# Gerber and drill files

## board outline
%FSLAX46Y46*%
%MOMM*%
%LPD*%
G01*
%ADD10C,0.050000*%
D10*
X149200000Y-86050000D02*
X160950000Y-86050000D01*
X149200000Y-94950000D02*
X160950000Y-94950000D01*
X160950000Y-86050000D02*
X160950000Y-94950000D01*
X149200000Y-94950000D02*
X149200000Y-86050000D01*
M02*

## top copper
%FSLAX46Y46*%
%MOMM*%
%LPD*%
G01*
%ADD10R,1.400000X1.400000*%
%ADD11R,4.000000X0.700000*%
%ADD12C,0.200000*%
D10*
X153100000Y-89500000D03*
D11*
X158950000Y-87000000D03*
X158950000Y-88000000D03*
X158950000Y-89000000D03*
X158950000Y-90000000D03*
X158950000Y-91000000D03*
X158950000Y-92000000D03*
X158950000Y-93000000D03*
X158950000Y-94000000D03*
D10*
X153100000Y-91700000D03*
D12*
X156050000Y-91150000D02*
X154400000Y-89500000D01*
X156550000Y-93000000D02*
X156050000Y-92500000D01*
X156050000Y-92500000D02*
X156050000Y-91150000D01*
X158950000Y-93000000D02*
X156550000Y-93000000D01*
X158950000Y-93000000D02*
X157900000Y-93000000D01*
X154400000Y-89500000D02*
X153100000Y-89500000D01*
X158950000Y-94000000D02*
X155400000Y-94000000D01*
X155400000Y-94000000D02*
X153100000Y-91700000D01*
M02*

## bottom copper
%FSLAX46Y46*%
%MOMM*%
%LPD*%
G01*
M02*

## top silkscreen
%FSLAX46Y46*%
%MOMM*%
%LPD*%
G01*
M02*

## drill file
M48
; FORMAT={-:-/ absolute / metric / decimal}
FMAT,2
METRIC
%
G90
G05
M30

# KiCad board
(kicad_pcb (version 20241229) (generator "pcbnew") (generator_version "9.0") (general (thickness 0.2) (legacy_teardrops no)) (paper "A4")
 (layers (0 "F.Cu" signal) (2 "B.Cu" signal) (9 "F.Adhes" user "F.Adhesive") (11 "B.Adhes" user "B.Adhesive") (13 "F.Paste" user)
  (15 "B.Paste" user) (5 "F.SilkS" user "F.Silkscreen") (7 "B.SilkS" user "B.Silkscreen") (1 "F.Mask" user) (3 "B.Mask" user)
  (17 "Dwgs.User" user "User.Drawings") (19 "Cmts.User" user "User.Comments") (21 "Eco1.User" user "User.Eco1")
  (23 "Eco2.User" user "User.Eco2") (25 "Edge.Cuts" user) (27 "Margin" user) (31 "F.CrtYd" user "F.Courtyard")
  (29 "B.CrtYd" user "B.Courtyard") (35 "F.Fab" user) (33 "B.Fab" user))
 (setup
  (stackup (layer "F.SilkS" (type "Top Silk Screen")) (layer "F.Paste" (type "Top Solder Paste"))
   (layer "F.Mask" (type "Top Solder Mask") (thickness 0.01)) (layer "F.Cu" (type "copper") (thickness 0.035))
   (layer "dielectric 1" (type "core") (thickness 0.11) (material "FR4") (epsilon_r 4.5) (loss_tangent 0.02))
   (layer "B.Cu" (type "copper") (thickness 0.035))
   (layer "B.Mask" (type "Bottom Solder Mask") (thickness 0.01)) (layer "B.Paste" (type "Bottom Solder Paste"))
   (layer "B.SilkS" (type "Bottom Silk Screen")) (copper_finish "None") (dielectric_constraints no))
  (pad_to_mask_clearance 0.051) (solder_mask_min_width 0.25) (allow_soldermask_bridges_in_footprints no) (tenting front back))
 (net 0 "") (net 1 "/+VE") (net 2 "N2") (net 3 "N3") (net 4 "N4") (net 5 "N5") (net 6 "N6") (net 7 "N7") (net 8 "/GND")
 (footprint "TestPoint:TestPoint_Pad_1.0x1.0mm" (layer "F.Cu") (at 153.1 89.3)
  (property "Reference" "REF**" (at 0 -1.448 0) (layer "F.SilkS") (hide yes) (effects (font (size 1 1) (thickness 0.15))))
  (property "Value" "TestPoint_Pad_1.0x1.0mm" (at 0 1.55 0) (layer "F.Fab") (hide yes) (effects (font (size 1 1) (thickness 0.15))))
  (pad "1" smd rect (at 0 0.2) (size 1.4 1.4) (layers "F.Cu" "F.Mask") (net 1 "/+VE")))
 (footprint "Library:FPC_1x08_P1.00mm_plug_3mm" (layer "F.Cu") (at 156.95 90.5)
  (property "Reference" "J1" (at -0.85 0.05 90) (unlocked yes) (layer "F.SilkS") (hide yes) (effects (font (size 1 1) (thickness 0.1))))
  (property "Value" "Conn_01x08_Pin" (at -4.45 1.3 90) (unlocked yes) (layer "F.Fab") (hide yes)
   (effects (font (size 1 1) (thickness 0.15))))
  (pad "1" connect rect (at 2 -3.5) (size 4 0.7) (layers "F.Cu" "F.Mask") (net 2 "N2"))
  (pad "2" connect rect (at 2 -2.5) (size 4 0.7) (layers "F.Cu" "F.Mask") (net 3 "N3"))
  (pad "3" connect rect (at 2 -1.5) (size 4 0.7) (layers "F.Cu" "F.Mask") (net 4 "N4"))
  (pad "4" connect rect (at 2 -0.5) (size 4 0.7) (layers "F.Cu" "F.Mask") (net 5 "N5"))
  (pad "5" connect rect (at 2 0.5) (size 4 0.7) (layers "F.Cu" "F.Mask") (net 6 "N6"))
  (pad "6" connect rect (at 2 1.5) (size 4 0.7) (layers "F.Cu" "F.Mask") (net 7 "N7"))
  (pad "7" connect rect (at 2 2.5) (size 4 0.7) (layers "F.Cu" "F.Mask") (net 1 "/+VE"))
  (pad "8" connect rect (at 2 3.5) (size 4 0.7) (layers "F.Cu" "F.Mask") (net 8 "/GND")))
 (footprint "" (layer "F.Cu") (at 153.1 91.7)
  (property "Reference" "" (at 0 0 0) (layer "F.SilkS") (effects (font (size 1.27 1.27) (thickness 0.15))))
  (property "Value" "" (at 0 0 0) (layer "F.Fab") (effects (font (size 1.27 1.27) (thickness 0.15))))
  (pad "1" smd rect (at 0 0) (size 1.4 1.4) (layers "F.Cu" "F.Mask") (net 8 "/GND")))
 (gr_line (start 149.2 86.05) (end 160.95 86.05) (stroke (width 0.05) (type default)) (layer "Edge.Cuts"))
 (gr_line (start 149.2 94.95) (end 160.95 94.95) (stroke (width 0.05) (type default)) (layer "Edge.Cuts"))
 (gr_line (start 160.95 86.05) (end 160.95 94.95) (stroke (width 0.05) (type default)) (layer "Edge.Cuts"))
 (gr_line (start 149.2 94.95) (end 149.2 86.05) (stroke (width 0.05) (type default)) (layer "Edge.Cuts"))
 (segment (start 156.05 91.15) (end 154.4 89.5) (width 0.2) (layer "F.Cu") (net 1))
 (segment (start 156.55 93) (end 156.05 92.5) (width 0.2) (layer "F.Cu") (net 1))
 (segment (start 156.05 92.5) (end 156.05 91.15) (width 0.2) (layer "F.Cu") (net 1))
 (segment (start 158.95 93) (end 156.55 93) (width 0.2) (layer "F.Cu") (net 1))
 (segment (start 158.95 93) (end 157.9 93) (width 0.2) (layer "F.Cu") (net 1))
 (segment (start 154.4 89.5) (end 153.1 89.5) (width 0.2) (layer "F.Cu") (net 1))
 (segment (start 158.95 94) (end 155.4 94) (width 0.2) (layer "F.Cu") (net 8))
 (segment (start 155.4 94) (end 153.1 91.7) (width 0.2) (layer "F.Cu") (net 8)))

